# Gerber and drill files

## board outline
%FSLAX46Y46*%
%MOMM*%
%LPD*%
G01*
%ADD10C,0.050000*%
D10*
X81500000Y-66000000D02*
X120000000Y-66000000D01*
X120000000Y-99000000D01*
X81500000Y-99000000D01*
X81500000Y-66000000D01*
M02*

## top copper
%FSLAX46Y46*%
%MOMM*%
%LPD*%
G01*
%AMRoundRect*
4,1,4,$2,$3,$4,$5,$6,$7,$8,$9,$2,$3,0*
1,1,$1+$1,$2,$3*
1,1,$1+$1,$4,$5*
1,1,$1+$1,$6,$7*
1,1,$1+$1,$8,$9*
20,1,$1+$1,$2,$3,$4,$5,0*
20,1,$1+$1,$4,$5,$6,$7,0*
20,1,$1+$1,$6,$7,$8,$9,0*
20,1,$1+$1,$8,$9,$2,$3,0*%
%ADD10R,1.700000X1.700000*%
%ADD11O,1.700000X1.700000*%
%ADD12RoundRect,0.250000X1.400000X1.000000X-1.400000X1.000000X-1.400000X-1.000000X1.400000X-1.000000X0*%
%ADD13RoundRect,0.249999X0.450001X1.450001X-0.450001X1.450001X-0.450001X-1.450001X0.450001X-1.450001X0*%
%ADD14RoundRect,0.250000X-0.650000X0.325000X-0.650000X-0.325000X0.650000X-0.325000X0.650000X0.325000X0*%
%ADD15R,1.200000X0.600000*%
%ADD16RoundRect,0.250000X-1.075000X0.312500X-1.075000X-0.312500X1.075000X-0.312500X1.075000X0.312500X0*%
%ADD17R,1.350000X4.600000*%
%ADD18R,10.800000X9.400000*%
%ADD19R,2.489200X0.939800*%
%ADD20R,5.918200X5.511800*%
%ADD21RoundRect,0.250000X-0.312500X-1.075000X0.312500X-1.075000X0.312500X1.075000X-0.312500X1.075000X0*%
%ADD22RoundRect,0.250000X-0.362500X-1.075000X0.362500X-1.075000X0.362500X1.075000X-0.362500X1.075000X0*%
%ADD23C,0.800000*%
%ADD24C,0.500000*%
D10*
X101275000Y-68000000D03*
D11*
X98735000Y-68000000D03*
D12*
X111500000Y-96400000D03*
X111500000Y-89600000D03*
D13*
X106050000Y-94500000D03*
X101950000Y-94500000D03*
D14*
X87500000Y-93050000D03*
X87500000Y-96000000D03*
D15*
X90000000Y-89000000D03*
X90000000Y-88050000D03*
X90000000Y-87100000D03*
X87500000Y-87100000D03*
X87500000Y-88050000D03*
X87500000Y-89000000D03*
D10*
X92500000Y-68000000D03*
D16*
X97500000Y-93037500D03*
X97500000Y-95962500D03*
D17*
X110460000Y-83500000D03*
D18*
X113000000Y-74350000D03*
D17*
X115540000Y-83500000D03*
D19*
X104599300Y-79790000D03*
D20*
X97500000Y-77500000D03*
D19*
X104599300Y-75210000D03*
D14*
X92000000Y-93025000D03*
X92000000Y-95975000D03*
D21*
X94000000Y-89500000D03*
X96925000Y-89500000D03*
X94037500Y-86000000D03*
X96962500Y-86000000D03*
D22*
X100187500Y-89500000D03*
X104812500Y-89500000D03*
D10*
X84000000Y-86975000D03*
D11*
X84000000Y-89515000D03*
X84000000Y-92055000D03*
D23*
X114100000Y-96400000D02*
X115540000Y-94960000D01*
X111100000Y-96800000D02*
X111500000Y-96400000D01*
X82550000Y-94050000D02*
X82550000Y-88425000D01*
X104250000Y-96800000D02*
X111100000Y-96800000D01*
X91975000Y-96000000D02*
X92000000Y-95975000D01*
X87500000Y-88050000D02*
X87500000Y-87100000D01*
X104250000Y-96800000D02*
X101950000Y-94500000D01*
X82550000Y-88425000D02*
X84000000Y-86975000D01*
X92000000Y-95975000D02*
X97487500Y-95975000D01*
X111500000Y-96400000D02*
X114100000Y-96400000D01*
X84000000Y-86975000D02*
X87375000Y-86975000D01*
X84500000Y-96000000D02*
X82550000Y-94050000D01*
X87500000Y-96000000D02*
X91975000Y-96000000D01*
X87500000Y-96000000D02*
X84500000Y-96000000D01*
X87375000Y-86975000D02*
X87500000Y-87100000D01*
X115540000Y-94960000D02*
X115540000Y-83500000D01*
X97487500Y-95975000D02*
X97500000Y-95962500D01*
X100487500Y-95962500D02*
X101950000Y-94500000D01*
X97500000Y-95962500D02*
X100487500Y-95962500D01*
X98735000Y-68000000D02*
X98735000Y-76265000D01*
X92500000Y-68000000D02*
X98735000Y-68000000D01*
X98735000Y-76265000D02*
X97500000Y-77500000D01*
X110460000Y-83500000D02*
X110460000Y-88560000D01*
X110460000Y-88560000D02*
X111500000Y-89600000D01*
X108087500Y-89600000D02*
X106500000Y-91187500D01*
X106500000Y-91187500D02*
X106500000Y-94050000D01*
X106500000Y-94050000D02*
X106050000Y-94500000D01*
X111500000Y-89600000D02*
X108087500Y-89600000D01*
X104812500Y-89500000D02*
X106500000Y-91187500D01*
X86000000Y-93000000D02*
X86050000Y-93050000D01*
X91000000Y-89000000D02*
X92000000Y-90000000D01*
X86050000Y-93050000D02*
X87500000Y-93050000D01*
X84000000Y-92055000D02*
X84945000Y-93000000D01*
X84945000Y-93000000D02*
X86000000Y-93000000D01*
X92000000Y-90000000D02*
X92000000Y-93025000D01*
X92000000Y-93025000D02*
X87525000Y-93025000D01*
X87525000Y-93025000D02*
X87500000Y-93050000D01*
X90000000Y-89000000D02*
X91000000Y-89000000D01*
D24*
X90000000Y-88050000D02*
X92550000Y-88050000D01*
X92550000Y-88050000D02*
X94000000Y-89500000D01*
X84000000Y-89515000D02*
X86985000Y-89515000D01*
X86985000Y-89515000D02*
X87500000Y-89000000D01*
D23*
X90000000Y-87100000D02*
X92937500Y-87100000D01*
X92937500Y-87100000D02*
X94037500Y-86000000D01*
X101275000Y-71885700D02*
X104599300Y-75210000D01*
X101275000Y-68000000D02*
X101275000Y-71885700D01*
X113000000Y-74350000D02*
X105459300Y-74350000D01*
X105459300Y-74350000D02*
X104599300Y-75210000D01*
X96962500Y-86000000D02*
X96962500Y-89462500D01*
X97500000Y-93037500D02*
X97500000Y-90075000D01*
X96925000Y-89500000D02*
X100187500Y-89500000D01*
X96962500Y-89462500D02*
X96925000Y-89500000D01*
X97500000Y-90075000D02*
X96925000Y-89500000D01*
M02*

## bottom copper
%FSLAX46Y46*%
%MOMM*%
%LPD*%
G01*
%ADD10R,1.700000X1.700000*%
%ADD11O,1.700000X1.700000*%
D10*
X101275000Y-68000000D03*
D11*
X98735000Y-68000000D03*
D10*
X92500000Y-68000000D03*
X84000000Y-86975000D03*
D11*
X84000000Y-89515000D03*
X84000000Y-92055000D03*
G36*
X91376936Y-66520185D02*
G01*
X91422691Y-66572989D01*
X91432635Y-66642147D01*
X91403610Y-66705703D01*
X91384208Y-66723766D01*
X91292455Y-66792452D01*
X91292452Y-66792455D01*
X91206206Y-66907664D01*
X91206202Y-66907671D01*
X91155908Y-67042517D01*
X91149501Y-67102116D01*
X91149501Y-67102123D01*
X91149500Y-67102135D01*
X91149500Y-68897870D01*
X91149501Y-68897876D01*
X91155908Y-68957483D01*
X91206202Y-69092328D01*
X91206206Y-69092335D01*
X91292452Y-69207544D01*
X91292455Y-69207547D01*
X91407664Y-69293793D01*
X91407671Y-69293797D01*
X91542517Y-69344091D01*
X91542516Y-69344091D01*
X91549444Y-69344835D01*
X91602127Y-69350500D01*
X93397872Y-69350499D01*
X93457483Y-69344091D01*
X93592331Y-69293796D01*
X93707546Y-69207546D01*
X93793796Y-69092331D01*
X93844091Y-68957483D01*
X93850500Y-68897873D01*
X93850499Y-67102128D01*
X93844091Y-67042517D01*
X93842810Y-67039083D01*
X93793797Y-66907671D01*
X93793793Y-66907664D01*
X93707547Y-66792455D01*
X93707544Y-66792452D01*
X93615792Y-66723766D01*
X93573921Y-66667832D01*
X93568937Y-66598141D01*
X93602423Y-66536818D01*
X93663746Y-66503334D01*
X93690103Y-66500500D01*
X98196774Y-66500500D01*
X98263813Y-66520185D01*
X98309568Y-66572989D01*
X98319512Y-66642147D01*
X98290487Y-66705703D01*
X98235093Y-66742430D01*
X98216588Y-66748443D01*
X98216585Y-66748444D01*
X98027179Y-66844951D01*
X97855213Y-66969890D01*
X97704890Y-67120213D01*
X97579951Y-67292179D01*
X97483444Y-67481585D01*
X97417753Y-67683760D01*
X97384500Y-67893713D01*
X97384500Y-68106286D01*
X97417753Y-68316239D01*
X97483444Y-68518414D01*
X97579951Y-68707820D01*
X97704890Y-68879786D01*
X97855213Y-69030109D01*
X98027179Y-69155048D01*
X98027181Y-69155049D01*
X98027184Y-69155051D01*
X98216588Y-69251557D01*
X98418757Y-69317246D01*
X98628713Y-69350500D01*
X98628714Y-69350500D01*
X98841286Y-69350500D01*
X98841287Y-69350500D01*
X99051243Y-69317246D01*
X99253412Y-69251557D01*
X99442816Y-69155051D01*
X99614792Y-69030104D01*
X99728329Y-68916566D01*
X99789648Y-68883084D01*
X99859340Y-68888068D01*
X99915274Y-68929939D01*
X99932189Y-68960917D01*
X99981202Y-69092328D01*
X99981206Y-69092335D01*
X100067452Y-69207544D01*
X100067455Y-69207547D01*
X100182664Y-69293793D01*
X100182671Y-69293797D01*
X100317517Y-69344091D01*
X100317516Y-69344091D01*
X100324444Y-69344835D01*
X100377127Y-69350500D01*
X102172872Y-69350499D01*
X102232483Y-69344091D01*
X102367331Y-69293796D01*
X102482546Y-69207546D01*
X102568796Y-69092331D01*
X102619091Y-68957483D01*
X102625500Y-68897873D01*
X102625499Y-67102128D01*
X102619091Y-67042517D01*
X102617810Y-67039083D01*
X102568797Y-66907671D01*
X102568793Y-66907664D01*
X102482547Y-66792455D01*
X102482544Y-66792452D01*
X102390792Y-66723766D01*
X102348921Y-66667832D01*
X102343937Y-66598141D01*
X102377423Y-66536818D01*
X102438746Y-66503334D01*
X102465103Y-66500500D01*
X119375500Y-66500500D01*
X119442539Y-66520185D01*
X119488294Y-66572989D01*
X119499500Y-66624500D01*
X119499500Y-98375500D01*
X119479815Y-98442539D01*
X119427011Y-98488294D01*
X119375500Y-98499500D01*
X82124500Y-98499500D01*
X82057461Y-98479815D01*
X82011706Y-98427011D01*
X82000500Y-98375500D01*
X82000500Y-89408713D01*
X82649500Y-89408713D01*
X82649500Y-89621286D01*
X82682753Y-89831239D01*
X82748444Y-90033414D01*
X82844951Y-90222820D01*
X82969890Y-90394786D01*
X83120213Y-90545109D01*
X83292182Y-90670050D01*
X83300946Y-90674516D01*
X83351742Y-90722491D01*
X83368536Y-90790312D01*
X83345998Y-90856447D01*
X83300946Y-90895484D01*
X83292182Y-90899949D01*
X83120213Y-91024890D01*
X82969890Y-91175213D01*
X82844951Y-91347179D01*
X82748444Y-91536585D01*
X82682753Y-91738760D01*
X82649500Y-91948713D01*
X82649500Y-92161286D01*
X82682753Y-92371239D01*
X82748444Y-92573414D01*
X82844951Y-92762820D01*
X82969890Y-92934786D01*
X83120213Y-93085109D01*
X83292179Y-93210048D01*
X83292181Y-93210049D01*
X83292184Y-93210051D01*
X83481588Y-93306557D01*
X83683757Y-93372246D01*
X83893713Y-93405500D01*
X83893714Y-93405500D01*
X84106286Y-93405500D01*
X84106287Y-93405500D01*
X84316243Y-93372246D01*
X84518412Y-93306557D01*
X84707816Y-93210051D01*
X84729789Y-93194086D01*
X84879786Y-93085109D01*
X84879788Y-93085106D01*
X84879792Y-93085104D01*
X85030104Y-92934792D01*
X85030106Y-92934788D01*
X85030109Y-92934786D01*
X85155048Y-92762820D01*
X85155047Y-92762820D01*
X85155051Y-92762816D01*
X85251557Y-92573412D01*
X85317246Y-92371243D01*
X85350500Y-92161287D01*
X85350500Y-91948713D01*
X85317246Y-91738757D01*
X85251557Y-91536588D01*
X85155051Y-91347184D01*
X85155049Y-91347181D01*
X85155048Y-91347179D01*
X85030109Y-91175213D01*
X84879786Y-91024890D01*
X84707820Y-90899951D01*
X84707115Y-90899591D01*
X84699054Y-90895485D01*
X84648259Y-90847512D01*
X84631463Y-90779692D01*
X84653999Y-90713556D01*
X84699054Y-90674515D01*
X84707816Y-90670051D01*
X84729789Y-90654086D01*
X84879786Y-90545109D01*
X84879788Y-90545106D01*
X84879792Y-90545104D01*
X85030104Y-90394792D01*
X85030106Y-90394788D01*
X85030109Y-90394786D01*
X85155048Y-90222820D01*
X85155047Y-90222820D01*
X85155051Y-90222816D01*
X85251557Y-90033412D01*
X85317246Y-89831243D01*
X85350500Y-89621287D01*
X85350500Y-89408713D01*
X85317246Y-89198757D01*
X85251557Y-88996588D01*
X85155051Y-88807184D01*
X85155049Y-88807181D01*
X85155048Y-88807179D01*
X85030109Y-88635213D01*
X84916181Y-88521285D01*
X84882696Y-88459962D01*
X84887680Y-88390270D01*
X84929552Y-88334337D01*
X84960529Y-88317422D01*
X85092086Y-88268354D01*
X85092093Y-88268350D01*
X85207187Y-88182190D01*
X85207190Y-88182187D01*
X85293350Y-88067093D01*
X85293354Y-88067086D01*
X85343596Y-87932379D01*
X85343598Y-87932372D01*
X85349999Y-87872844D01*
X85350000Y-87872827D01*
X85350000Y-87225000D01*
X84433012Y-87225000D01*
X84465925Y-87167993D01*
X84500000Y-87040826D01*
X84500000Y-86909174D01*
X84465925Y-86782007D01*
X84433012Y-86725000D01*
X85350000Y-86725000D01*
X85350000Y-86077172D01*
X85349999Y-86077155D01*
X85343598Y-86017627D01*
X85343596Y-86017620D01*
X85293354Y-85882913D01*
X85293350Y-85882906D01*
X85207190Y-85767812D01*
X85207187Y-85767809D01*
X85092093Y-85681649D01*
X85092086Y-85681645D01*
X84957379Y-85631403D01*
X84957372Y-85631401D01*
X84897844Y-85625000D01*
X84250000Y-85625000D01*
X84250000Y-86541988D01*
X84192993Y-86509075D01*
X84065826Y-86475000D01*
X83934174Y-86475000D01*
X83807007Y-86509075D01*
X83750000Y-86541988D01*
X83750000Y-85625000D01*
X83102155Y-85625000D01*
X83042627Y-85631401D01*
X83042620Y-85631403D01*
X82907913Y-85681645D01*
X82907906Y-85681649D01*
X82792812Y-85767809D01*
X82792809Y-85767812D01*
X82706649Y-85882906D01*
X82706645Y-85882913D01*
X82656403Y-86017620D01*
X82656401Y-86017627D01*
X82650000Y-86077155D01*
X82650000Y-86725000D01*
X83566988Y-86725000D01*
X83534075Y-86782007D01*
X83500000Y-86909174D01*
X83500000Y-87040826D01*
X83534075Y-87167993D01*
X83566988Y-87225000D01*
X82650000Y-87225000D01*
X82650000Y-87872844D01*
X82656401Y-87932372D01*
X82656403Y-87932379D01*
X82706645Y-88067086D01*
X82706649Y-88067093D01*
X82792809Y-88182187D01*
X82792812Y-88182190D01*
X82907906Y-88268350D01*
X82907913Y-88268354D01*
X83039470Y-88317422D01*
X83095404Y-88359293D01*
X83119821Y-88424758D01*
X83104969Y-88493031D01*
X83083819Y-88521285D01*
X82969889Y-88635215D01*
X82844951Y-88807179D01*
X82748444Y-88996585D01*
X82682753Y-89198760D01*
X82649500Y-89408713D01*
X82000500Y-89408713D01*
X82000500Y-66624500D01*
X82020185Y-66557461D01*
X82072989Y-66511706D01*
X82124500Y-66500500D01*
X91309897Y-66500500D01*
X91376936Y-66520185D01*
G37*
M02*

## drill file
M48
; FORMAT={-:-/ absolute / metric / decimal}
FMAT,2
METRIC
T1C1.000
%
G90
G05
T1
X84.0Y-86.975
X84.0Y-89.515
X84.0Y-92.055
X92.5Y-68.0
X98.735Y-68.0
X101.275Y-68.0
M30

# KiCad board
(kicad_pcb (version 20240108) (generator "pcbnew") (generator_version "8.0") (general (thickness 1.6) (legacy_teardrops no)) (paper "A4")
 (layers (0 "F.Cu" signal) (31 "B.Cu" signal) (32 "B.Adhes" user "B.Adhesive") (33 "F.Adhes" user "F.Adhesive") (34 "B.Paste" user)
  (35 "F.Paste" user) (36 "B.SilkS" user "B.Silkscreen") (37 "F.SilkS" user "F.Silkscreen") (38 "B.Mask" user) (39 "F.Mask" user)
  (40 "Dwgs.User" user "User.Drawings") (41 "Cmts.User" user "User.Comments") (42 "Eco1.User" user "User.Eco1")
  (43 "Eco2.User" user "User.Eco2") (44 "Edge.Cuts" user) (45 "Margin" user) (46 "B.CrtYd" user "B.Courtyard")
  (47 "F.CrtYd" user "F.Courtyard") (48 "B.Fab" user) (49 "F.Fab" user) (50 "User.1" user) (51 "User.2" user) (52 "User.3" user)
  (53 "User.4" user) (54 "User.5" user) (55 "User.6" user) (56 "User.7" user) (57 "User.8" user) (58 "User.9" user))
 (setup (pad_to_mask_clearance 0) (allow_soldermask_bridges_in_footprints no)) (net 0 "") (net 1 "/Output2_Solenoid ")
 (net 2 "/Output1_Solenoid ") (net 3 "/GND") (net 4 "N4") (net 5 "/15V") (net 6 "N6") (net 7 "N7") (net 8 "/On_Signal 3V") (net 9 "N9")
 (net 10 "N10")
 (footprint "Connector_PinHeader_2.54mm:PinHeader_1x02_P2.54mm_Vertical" (layer "F.Cu") (at 101.275 68 -90)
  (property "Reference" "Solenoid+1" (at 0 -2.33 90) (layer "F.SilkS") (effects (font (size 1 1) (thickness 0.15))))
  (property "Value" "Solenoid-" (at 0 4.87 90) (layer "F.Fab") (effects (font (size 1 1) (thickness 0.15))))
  (pad "1" thru_hole rect (at 0 0 270) (size 1.7 1.7) (drill 1) (layers "*.Cu" "*.Mask") (remove_unused_layers no)
   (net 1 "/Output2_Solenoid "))
  (pad "2" thru_hole oval (at 0 2.54 270) (size 1.7 1.7) (drill 1) (layers "*.Cu" "*.Mask") (remove_unused_layers no)
   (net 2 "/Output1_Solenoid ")))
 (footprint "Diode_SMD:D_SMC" (layer "F.Cu") (at 111.5 93 90)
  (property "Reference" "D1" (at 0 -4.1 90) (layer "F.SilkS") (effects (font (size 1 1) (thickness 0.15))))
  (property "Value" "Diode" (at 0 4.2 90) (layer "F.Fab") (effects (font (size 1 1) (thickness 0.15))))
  (pad "1" smd roundrect (at -3.4 0 180) (size 3.3 2.5) (layers "F.Cu" "F.Paste" "F.Mask") (roundrect_rratio 0.1) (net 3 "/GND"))
  (pad "2" smd roundrect (at 3.4 0 180) (size 3.3 2.5) (layers "F.Cu" "F.Paste" "F.Mask") (roundrect_rratio 0.1) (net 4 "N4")))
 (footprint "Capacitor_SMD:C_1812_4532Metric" (layer "F.Cu") (at 104 94.5 180)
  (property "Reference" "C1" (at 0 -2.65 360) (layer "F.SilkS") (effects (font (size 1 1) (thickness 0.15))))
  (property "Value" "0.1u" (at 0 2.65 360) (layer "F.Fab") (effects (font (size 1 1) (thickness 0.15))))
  (pad "1" smd roundrect (at -2.05 0 180) (size 1.4 3.4) (layers "F.Cu" "F.Paste" "F.Mask") (roundrect_rratio 0.178571) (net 4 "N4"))
  (pad "2" smd roundrect (at 2.05 0 180) (size 1.4 3.4) (layers "F.Cu" "F.Paste" "F.Mask") (roundrect_rratio 0.178571) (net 3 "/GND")))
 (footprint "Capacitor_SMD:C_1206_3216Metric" (layer "F.Cu") (at 87.5 94.525 -90)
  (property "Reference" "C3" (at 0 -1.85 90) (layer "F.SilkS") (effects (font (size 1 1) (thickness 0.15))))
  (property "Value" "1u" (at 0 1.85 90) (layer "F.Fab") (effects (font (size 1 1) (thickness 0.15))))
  (pad "1" smd roundrect (at -1.475 0 270) (size 1.15 1.8) (layers "F.Cu" "F.Paste" "F.Mask") (roundrect_rratio 0.217391) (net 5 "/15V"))
  (pad "2" smd roundrect (at 1.475 0 270) (size 1.15 1.8) (layers "F.Cu" "F.Paste" "F.Mask") (roundrect_rratio 0.217391) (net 3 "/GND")))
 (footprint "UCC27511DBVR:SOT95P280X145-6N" (layer "F.Cu") (at 88.75 88.05 180)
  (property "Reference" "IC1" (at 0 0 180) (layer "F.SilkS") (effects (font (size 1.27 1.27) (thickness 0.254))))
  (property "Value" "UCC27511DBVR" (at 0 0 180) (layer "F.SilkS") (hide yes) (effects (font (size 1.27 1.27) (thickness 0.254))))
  (pad "1" smd rect (at -1.25 -0.95 270) (size 0.6 1.2) (layers "F.Cu" "F.Paste" "F.Mask") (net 5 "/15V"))
  (pad "2" smd rect (at -1.25 0 270) (size 0.6 1.2) (layers "F.Cu" "F.Paste" "F.Mask") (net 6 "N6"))
  (pad "3" smd rect (at -1.25 0.95 270) (size 0.6 1.2) (layers "F.Cu" "F.Paste" "F.Mask") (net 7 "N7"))
  (pad "4" smd rect (at 1.25 0.95 270) (size 0.6 1.2) (layers "F.Cu" "F.Paste" "F.Mask") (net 3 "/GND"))
  (pad "5" smd rect (at 1.25 0 270) (size 0.6 1.2) (layers "F.Cu" "F.Paste" "F.Mask") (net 3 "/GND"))
  (pad "6" smd rect (at 1.25 -0.95 270) (size 0.6 1.2) (layers "F.Cu" "F.Paste" "F.Mask") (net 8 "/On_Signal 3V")))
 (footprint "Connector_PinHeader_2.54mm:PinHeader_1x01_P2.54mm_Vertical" (layer "F.Cu") (at 92.5 68)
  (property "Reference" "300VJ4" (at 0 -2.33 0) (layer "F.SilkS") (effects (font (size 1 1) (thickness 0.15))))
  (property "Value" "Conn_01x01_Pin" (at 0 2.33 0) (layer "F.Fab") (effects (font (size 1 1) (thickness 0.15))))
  (pad "1" thru_hole rect (at 0 0) (size 1.7 1.7) (drill 1) (layers "*.Cu" "*.Mask") (remove_unused_layers no) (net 2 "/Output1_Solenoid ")))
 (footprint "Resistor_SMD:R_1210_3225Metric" (layer "F.Cu") (at 97.5 94.5 -90)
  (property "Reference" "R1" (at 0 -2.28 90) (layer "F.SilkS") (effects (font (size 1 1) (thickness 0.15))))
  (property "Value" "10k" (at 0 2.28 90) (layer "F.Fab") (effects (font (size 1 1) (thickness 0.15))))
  (pad "1" smd roundrect (at -1.4625 0 270) (size 1.125 2.65) (layers "F.Cu" "F.Paste" "F.Mask") (roundrect_rratio 0.222222) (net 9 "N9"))
  (pad "2" smd roundrect (at 1.4625 0 270) (size 1.125 2.65) (layers "F.Cu" "F.Paste" "F.Mask") (roundrect_rratio 0.222222) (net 3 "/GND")))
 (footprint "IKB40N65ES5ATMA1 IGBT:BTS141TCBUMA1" (layer "F.Cu") (at 113 78.425)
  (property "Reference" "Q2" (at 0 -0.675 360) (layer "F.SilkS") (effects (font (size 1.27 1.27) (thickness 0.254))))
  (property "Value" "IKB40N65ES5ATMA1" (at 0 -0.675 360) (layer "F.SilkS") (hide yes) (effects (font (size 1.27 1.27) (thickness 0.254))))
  (pad "1" smd rect (at -2.54 5.075) (size 1.35 4.6) (layers "F.Cu" "F.Paste" "F.Mask") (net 4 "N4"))
  (pad "2" smd rect (at 0 -4.075 90) (size 9.4 10.8) (layers "F.Cu" "F.Paste" "F.Mask") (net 1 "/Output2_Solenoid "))
  (pad "3" smd rect (at 2.54 5.075) (size 1.35 4.6) (layers "F.Cu" "F.Paste" "F.Mask") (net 3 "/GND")))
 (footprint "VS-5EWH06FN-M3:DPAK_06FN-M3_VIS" (layer "F.Cu") (at 99.4558 77.5 90)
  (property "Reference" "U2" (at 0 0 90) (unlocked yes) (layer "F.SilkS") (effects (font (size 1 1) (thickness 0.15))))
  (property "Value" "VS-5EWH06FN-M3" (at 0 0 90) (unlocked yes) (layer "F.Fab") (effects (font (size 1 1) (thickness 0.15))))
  (pad "1" smd rect (at -2.29 5.1435 90) (size 0.9398 2.4892) (layers "F.Cu" "F.Paste" "F.Mask") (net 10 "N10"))
  (pad "2" smd rect (at 0 -1.9558 90) (size 5.5118 5.9182) (layers "F.Cu" "F.Paste" "F.Mask") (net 2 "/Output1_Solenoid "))
  (pad "3" smd rect (at 2.29 5.1435 90) (size 0.9398 2.4892) (layers "F.Cu" "F.Paste" "F.Mask") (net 1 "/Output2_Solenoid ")))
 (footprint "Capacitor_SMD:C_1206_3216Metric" (layer "F.Cu") (at 92 94.5 -90)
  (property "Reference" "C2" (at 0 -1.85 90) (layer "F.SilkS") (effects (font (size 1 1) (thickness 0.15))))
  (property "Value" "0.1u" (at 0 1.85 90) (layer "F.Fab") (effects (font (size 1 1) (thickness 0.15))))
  (pad "1" smd roundrect (at -1.475 0 270) (size 1.15 1.8) (layers "F.Cu" "F.Paste" "F.Mask") (roundrect_rratio 0.217391) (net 5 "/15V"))
  (pad "2" smd roundrect (at 1.475 0 270) (size 1.15 1.8) (layers "F.Cu" "F.Paste" "F.Mask") (roundrect_rratio 0.217391) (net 3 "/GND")))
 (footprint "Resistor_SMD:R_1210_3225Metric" (layer "F.Cu") (at 95.4625 89.5)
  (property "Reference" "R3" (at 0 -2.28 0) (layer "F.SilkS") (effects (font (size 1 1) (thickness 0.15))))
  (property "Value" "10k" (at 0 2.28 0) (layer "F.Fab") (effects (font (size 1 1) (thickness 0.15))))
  (pad "1" smd roundrect (at -1.4625 0) (size 1.125 2.65) (layers "F.Cu" "F.Paste" "F.Mask") (roundrect_rratio 0.222222) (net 6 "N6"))
  (pad "2" smd roundrect (at 1.4625 0) (size 1.125 2.65) (layers "F.Cu" "F.Paste" "F.Mask") (roundrect_rratio 0.222222) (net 9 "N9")))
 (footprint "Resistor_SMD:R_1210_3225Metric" (layer "F.Cu") (at 95.5 86)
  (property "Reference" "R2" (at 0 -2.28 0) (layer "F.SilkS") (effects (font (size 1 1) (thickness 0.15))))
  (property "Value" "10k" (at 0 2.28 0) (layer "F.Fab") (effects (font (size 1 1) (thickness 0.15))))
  (pad "1" smd roundrect (at -1.4625 0) (size 1.125 2.65) (layers "F.Cu" "F.Paste" "F.Mask") (roundrect_rratio 0.222222) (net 7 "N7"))
  (pad "2" smd roundrect (at 1.4625 0) (size 1.125 2.65) (layers "F.Cu" "F.Paste" "F.Mask") (roundrect_rratio 0.222222) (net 9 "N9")))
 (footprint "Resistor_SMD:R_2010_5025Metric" (layer "F.Cu") (at 102.5 89.5)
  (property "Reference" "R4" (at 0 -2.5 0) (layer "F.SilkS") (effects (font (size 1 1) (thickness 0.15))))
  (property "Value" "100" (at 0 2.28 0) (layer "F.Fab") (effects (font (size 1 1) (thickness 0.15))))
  (pad "1" smd roundrect (at -2.3125 0) (size 1.225 2.65) (layers "F.Cu" "F.Paste" "F.Mask") (roundrect_rratio 0.204082) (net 9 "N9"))
  (pad "2" smd roundrect (at 2.3125 0) (size 1.225 2.65) (layers "F.Cu" "F.Paste" "F.Mask") (roundrect_rratio 0.204082) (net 4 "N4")))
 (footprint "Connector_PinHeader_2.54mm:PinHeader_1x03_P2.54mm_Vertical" (layer "F.Cu") (at 84 86.975)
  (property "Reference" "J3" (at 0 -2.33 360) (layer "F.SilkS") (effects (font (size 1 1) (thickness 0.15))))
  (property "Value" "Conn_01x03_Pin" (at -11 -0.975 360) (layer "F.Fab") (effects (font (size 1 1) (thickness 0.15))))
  (pad "1" thru_hole rect (at 0 0) (size 1.7 1.7) (drill 1) (layers "*.Cu" "*.Mask") (remove_unused_layers no) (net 3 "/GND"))
  (pad "2" thru_hole oval (at 0 2.54) (size 1.7 1.7) (drill 1) (layers "*.Cu" "*.Mask") (remove_unused_layers no) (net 8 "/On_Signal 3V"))
  (pad "3" thru_hole oval (at 0 5.08) (size 1.7 1.7) (drill 1) (layers "*.Cu" "*.Mask") (remove_unused_layers no) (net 5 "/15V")))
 (gr_rect (start 81.5 66) (end 120 99) (stroke (width 0.05) (type default)) (fill none) (layer "Edge.Cuts"))
 (segment (start 114.1 96.4) (end 115.54 94.96) (width 0.8) (layer "F.Cu") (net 3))
 (segment (start 111.1 96.8) (end 111.5 96.4) (width 0.8) (layer "F.Cu") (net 3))
 (segment (start 82.55 94.05) (end 82.55 88.425) (width 0.8) (layer "F.Cu") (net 3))
 (segment (start 104.25 96.8) (end 111.1 96.8) (width 0.8) (layer "F.Cu") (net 3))
 (segment (start 91.975 96) (end 92 95.975) (width 0.8) (layer "F.Cu") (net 3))
 (segment (start 87.5 88.05) (end 87.5 87.1) (width 0.8) (layer "F.Cu") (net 3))
 (segment (start 104.25 96.8) (end 101.95 94.5) (width 0.8) (layer "F.Cu") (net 3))
 (segment (start 82.55 88.425) (end 84 86.975) (width 0.8) (layer "F.Cu") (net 3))
 (segment (start 92 95.975) (end 97.4875 95.975) (width 0.8) (layer "F.Cu") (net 3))
 (segment (start 111.5 96.4) (end 114.1 96.4) (width 0.8) (layer "F.Cu") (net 3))
 (segment (start 84 86.975) (end 87.375 86.975) (width 0.8) (layer "F.Cu") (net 3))
 (segment (start 84.5 96) (end 82.55 94.05) (width 0.8) (layer "F.Cu") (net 3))
 (segment (start 87.5 96) (end 91.975 96) (width 0.8) (layer "F.Cu") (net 3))
 (segment (start 87.5 96) (end 84.5 96) (width 0.8) (layer "F.Cu") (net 3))
 (segment (start 87.375 86.975) (end 87.5 87.1) (width 0.8) (layer "F.Cu") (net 3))
 (segment (start 115.54 94.96) (end 115.54 83.5) (width 0.8) (layer "F.Cu") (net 3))
 (segment (start 97.4875 95.975) (end 97.5 95.9625) (width 0.8) (layer "F.Cu") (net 3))
 (segment (start 100.4875 95.9625) (end 101.95 94.5) (width 0.8) (layer "F.Cu") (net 3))
 (segment (start 97.5 95.9625) (end 100.4875 95.9625) (width 0.8) (layer "F.Cu") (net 3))
 (segment (start 98.735 68) (end 98.735 76.265) (width 0.8) (layer "F.Cu") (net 2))
 (segment (start 92.5 68) (end 98.735 68) (width 0.8) (layer "F.Cu") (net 2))
 (segment (start 98.735 76.265) (end 97.5 77.5) (width 0.8) (layer "F.Cu") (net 2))
 (segment (start 110.46 83.5) (end 110.46 88.56) (width 0.8) (layer "F.Cu") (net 4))
 (segment (start 110.46 88.56) (end 111.5 89.6) (width 0.8) (layer "F.Cu") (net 4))
 (segment (start 108.0875 89.6) (end 106.5 91.1875) (width 0.8) (layer "F.Cu") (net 4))
 (segment (start 106.5 91.1875) (end 106.5 94.05) (width 0.8) (layer "F.Cu") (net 4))
 (segment (start 106.5 94.05) (end 106.05 94.5) (width 0.8) (layer "F.Cu") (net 4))
 (segment (start 111.5 89.6) (end 108.0875 89.6) (width 0.8) (layer "F.Cu") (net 4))
 (segment (start 104.8125 89.5) (end 106.5 91.1875) (width 0.8) (layer "F.Cu") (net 4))
 (segment (start 86 93) (end 86.05 93.05) (width 0.8) (layer "F.Cu") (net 5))
 (segment (start 91 89) (end 92 90) (width 0.8) (layer "F.Cu") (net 5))
 (segment (start 86.05 93.05) (end 87.5 93.05) (width 0.8) (layer "F.Cu") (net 5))
 (segment (start 84 92.055) (end 84.945 93) (width 0.8) (layer "F.Cu") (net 5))
 (segment (start 84.945 93) (end 86 93) (width 0.8) (layer "F.Cu") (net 5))
 (segment (start 92 90) (end 92 93.025) (width 0.8) (layer "F.Cu") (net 5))
 (segment (start 92 93.025) (end 87.525 93.025) (width 0.8) (layer "F.Cu") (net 5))
 (segment (start 87.525 93.025) (end 87.5 93.05) (width 0.8) (layer "F.Cu") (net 5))
 (segment (start 90 89) (end 91 89) (width 0.8) (layer "F.Cu") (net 5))
 (segment (start 90 88.05) (end 92.55 88.05) (width 0.5) (layer "F.Cu") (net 6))
 (segment (start 92.55 88.05) (end 94 89.5) (width 0.5) (layer "F.Cu") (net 6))
 (segment (start 84 89.515) (end 86.985 89.515) (width 0.5) (layer "F.Cu") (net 8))
 (segment (start 86.985 89.515) (end 87.5 89) (width 0.5) (layer "F.Cu") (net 8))
 (segment (start 90 87.1) (end 92.9375 87.1) (width 0.8) (layer "F.Cu") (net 7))
 (segment (start 92.9375 87.1) (end 94.0375 86) (width 0.8) (layer "F.Cu") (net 7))
 (segment (start 101.275 71.8857) (end 104.5993 75.21) (width 0.8) (layer "F.Cu") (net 1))
 (segment (start 101.275 68) (end 101.275 71.8857) (width 0.8) (layer "F.Cu") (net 1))
 (segment (start 113 74.35) (end 105.4593 74.35) (width 0.8) (layer "F.Cu") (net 1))
 (segment (start 105.4593 74.35) (end 104.5993 75.21) (width 0.8) (layer "F.Cu") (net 1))
 (segment (start 96.9625 86) (end 96.9625 89.4625) (width 0.8) (layer "F.Cu") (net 9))
 (segment (start 97.5 93.0375) (end 97.5 90.075) (width 0.8) (layer "F.Cu") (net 9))
 (segment (start 96.925 89.5) (end 100.1875 89.5) (width 0.8) (layer "F.Cu") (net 9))
 (segment (start 96.9625 89.4625) (end 96.925 89.5) (width 0.8) (layer "F.Cu") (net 9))
 (segment (start 97.5 90.075) (end 96.925 89.5) (width 0.8) (layer "F.Cu") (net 9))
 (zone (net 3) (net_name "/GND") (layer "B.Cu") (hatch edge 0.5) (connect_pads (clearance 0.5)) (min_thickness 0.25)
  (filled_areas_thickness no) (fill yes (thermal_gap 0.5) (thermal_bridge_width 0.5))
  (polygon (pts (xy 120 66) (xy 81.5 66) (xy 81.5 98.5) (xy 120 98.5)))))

